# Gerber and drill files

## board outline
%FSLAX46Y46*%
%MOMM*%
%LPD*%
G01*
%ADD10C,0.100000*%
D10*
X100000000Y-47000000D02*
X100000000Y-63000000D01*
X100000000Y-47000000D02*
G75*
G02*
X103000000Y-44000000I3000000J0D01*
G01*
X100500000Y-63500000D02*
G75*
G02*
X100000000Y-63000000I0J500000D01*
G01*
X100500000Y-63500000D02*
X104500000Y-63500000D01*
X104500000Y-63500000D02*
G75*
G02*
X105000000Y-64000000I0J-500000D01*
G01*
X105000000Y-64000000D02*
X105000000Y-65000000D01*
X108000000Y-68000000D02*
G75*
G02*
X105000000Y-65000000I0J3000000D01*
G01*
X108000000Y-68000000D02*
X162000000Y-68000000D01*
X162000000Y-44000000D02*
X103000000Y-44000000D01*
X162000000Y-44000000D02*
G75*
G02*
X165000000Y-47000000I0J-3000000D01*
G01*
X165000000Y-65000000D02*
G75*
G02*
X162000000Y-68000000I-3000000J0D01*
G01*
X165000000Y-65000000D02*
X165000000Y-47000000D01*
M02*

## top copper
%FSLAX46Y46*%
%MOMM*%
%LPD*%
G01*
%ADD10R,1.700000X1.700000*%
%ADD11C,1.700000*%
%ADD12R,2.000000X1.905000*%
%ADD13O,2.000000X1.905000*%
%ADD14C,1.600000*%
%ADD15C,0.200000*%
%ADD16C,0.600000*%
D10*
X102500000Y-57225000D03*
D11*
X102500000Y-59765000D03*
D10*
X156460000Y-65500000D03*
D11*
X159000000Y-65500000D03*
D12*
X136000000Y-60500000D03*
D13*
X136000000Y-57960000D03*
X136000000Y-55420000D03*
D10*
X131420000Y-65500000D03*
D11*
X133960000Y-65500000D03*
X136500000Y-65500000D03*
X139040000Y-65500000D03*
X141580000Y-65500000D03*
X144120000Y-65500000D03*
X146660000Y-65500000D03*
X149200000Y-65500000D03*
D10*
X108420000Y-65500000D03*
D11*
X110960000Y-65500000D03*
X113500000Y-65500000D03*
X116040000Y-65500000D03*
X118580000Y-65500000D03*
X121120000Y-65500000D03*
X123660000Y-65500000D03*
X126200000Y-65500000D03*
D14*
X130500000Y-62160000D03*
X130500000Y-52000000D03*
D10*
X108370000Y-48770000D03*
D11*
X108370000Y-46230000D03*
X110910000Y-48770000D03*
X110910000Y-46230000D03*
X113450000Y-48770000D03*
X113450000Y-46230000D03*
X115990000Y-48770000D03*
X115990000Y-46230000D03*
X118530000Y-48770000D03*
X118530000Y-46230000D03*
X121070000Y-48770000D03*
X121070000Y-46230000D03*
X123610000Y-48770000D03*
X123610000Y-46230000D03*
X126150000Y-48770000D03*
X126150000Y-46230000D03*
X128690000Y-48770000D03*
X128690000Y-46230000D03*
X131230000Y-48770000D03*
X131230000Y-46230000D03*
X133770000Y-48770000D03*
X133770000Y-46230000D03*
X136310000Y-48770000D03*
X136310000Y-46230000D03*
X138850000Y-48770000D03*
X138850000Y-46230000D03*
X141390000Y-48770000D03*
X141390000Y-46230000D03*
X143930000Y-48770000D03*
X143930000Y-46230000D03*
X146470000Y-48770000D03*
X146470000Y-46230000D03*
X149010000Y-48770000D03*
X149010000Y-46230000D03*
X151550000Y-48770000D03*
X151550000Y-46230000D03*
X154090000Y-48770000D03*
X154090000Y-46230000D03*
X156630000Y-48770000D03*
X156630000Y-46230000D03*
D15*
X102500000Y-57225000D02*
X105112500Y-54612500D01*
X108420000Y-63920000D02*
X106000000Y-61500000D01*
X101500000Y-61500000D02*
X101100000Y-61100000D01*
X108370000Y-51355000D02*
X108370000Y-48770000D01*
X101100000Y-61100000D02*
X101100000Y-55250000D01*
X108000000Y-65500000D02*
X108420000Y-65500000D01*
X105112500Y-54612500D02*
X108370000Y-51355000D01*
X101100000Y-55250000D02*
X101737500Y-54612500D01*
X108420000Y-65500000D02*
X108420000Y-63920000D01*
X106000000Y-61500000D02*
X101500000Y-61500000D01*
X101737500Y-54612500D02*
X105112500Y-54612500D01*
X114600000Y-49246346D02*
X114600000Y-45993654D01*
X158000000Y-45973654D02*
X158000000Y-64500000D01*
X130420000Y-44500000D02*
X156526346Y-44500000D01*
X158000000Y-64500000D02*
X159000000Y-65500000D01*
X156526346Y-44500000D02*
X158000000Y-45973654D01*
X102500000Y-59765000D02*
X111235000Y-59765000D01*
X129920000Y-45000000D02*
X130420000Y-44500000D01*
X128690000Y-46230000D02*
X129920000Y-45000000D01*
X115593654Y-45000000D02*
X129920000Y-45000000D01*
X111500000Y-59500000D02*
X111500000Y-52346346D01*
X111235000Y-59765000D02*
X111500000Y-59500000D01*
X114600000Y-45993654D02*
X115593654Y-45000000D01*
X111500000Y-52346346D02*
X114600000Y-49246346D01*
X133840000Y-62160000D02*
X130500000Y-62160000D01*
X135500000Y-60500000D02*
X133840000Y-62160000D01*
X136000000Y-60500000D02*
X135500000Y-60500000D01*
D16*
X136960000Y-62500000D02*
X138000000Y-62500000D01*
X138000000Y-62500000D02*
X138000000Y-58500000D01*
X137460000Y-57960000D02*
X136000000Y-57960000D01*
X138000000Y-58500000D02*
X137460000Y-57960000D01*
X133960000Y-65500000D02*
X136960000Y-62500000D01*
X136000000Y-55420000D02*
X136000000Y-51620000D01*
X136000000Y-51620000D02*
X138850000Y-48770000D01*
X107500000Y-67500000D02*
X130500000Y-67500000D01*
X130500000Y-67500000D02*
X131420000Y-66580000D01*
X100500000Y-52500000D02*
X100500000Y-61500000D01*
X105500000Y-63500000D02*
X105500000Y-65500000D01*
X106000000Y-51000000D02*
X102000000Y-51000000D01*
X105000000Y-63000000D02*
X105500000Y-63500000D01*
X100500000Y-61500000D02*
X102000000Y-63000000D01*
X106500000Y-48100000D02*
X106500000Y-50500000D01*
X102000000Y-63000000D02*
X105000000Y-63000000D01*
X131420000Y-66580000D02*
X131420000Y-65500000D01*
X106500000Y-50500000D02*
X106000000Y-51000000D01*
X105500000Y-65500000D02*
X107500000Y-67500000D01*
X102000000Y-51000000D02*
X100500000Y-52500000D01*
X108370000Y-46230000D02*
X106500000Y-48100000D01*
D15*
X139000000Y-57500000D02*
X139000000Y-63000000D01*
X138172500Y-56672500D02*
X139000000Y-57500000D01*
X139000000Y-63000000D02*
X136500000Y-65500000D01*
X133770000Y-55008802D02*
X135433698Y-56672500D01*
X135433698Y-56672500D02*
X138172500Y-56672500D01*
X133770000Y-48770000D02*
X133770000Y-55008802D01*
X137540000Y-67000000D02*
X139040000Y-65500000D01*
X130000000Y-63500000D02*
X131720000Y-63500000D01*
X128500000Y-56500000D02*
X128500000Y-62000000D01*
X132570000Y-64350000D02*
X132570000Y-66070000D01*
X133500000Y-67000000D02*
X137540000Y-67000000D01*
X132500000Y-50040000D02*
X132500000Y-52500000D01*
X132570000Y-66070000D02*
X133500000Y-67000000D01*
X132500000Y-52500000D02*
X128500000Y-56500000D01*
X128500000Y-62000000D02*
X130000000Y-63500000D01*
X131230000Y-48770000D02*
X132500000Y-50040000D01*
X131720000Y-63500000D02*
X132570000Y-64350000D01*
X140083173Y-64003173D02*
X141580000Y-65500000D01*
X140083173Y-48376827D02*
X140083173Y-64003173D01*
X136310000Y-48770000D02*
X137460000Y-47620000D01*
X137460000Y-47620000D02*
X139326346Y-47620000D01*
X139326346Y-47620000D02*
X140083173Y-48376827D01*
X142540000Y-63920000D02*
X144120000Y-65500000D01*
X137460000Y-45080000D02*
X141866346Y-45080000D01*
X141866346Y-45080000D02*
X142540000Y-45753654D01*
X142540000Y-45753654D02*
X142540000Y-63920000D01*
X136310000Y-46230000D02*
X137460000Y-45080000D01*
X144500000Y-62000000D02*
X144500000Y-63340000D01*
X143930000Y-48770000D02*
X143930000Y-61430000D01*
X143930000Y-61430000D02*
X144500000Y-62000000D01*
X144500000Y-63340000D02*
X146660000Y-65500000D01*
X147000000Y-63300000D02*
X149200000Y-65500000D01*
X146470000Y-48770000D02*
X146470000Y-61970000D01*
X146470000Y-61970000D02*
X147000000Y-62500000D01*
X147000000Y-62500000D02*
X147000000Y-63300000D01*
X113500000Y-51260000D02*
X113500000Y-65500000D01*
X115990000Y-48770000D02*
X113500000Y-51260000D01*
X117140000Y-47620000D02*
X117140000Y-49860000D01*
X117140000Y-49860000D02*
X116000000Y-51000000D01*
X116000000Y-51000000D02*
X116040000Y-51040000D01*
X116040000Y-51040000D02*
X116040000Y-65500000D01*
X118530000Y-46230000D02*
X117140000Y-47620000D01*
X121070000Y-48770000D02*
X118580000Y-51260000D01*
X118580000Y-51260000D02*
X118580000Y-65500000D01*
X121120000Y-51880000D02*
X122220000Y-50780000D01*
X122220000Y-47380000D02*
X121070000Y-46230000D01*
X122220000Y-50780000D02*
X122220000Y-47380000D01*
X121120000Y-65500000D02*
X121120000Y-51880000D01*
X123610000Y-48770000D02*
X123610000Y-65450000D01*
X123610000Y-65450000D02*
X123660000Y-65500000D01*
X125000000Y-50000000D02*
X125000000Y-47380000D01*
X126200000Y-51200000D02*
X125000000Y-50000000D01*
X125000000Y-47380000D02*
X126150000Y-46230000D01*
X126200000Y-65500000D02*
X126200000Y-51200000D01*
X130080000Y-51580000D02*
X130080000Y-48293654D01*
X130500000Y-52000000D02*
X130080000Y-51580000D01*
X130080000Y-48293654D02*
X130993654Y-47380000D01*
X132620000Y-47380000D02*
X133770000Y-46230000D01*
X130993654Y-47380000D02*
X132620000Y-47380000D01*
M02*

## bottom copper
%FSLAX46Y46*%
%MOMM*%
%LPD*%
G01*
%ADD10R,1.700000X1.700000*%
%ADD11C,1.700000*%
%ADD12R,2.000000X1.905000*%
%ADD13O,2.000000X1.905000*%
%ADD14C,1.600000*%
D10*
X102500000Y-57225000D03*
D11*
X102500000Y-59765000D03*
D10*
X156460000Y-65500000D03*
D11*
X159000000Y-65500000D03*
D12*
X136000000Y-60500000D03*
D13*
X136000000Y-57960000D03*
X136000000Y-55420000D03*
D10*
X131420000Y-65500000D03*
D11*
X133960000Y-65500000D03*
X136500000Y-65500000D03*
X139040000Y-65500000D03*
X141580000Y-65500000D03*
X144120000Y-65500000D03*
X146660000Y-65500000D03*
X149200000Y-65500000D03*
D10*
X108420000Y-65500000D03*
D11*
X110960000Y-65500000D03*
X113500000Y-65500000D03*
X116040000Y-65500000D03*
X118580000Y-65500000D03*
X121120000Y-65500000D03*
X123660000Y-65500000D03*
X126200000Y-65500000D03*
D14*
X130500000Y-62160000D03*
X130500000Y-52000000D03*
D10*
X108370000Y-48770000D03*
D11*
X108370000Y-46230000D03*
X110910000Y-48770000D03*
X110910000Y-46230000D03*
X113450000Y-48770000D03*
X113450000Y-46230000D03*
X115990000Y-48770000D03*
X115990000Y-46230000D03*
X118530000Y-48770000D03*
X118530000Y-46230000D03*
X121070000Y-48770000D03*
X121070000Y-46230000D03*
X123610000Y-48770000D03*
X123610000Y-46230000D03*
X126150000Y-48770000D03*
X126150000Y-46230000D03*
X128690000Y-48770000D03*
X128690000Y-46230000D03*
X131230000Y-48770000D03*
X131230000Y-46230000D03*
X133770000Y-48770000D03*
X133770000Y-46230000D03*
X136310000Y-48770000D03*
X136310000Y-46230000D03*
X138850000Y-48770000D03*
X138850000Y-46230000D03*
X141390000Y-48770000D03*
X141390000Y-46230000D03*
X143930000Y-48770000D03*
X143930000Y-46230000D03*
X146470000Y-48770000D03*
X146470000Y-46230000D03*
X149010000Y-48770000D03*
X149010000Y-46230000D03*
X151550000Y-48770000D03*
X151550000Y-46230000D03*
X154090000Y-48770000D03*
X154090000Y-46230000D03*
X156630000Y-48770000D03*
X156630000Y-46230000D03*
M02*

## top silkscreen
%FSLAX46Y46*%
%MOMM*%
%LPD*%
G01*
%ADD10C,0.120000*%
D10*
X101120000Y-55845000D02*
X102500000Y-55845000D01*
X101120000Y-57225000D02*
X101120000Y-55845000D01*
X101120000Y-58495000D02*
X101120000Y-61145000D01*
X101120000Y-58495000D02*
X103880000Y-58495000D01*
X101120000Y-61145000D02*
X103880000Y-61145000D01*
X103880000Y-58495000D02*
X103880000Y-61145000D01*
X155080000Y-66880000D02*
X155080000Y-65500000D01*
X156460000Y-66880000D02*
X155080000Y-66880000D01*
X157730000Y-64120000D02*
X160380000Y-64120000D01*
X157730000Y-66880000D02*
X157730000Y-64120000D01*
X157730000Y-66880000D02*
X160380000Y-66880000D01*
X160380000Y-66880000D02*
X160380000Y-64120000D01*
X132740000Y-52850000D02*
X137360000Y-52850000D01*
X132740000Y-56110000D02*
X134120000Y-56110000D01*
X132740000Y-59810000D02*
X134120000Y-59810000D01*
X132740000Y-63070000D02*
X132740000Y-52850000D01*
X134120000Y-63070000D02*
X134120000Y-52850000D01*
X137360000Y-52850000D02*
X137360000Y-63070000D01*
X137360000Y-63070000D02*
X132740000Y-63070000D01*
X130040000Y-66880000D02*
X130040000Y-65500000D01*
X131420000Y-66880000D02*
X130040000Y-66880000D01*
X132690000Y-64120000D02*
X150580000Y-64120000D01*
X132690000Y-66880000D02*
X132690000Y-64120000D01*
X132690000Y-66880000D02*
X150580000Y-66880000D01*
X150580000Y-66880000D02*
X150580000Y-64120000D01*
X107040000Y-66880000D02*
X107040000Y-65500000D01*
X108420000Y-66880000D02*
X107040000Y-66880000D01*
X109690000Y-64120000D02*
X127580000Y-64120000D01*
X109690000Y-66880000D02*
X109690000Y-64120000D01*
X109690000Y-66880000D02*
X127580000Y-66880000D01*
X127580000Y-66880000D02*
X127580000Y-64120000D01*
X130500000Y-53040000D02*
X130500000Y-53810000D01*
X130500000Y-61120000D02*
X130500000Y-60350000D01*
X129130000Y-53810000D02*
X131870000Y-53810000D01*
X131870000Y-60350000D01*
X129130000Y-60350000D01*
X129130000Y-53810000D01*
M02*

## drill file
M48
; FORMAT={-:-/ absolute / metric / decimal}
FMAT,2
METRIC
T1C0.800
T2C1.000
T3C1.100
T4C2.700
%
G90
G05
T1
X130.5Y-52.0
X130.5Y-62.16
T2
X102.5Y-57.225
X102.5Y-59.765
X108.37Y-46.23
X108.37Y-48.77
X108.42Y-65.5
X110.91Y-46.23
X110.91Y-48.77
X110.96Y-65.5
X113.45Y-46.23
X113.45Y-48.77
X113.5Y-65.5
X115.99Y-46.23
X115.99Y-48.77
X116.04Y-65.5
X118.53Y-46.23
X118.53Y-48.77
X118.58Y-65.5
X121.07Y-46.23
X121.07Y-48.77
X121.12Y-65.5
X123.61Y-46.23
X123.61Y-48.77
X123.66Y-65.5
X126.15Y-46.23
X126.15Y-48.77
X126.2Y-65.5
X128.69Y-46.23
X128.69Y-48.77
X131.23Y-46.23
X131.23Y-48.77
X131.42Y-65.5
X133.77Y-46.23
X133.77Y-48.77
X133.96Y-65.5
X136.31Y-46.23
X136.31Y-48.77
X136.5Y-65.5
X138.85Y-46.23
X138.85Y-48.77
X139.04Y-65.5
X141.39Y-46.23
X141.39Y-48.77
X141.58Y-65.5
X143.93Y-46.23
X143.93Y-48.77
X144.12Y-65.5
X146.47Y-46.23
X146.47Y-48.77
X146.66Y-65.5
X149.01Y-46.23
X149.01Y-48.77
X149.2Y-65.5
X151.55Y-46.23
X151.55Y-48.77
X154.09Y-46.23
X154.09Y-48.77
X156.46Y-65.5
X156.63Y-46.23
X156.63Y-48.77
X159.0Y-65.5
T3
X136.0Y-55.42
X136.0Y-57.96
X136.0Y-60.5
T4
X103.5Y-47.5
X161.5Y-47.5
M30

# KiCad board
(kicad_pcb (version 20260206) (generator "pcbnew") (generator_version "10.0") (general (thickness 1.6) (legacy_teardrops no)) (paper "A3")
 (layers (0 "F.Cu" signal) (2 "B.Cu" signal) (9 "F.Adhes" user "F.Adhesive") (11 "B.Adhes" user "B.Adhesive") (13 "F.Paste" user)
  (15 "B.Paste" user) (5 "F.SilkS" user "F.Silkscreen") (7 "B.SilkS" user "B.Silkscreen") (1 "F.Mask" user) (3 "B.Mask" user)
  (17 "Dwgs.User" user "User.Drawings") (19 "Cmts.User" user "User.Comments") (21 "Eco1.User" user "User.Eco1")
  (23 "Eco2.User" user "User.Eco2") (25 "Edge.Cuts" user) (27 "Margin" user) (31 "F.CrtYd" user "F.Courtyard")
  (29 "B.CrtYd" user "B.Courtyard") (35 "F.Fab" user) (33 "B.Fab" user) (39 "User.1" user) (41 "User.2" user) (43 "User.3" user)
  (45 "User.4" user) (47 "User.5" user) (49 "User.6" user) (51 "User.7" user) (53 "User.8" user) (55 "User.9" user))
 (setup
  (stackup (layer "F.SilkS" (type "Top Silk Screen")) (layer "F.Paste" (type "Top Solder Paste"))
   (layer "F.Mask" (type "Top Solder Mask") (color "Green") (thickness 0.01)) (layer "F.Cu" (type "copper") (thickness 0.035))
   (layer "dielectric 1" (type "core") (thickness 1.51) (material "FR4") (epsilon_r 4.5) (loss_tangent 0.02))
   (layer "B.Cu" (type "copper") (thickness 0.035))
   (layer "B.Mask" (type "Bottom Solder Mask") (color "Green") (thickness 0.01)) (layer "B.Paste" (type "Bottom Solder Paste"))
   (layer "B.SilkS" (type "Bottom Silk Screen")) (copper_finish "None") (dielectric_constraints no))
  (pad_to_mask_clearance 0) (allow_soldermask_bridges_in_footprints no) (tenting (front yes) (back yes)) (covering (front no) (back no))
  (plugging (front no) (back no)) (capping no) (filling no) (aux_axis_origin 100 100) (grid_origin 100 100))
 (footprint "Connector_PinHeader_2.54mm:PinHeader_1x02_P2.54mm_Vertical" (layer "F.Cu") (at 102.5 57.225)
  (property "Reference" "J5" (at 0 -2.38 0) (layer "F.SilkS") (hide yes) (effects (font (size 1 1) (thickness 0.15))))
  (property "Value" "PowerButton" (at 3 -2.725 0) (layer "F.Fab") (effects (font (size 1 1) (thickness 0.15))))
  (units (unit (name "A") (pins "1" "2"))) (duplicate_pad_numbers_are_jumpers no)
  (fp_line (start -1.38 -1.38) (end 0 -1.38) (stroke (width 0.12) (type solid)) (layer "F.SilkS"))
  (fp_line (start -1.38 0) (end -1.38 -1.38) (stroke (width 0.12) (type solid)) (layer "F.SilkS"))
  (fp_line (start -1.38 1.27) (end -1.38 3.92) (stroke (width 0.12) (type solid)) (layer "F.SilkS"))
  (fp_line (start -1.38 1.27) (end 1.38 1.27) (stroke (width 0.12) (type solid)) (layer "F.SilkS"))
  (fp_line (start -1.38 3.92) (end 1.38 3.92) (stroke (width 0.12) (type solid)) (layer "F.SilkS"))
  (fp_line (start 1.38 1.27) (end 1.38 3.92) (stroke (width 0.12) (type solid)) (layer "F.SilkS"))
  (pad "1" thru_hole rect (at 0 0) (size 1.7 1.7) (drill 1) (layers "*.Cu" "*.Mask") (remove_unused_layers no) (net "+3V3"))
  (pad "2" thru_hole circle (at 0 2.54) (size 1.7 1.7) (drill 1) (layers "*.Cu" "*.Mask") (remove_unused_layers no) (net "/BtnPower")))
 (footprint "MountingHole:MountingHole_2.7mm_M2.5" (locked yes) (layer "F.Cu") (at 161.5 47.5)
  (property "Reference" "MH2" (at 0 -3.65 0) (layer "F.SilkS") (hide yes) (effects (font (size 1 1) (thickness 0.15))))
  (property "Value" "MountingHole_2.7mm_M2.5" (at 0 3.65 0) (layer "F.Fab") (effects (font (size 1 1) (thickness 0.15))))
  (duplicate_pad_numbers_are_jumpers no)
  (pad "" np_thru_hole circle (at 0 0) (size 2.7 2.7) (drill 2.7) (layers "*.Cu" "*.Mask")))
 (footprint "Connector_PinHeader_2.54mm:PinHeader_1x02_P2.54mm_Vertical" (layer "F.Cu") (at 156.46 65.5 90)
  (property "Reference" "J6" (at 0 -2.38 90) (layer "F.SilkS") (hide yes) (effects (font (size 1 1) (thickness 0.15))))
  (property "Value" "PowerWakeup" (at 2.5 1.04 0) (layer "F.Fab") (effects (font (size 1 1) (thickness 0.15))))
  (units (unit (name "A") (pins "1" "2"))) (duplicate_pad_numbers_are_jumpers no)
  (fp_line (start -1.38 -1.38) (end 0 -1.38) (stroke (width 0.12) (type solid)) (layer "F.SilkS"))
  (fp_line (start -1.38 0) (end -1.38 -1.38) (stroke (width 0.12) (type solid)) (layer "F.SilkS"))
  (fp_line (start 1.38 1.27) (end 1.38 3.92) (stroke (width 0.12) (type solid)) (layer "F.SilkS"))
  (fp_line (start -1.38 1.27) (end 1.38 1.27) (stroke (width 0.12) (type solid)) (layer "F.SilkS"))
  (fp_line (start -1.38 1.27) (end -1.38 3.92) (stroke (width 0.12) (type solid)) (layer "F.SilkS"))
  (fp_line (start -1.38 3.92) (end 1.38 3.92) (stroke (width 0.12) (type solid)) (layer "F.SilkS"))
  (pad "1" thru_hole rect (at 0 0 90) (size 1.7 1.7) (drill 1) (layers "*.Cu" "*.Mask") (remove_unused_layers no)
   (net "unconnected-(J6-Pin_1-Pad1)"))
  (pad "2" thru_hole circle (at 0 2.54 90) (size 1.7 1.7) (drill 1) (layers "*.Cu" "*.Mask") (remove_unused_layers no) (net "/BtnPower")))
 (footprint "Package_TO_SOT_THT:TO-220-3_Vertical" (layer "F.Cu") (at 136 60.5 90)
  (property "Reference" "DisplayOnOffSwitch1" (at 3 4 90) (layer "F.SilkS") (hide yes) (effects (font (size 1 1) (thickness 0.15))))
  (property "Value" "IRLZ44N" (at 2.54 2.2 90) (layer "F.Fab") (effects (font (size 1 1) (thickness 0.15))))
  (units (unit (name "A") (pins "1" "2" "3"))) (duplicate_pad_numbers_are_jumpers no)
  (fp_line (start 7.65 -3.26) (end 7.65 1.36) (stroke (width 0.12) (type solid)) (layer "F.SilkS"))
  (fp_line (start 4.39 -3.26) (end 4.39 -1.88) (stroke (width 0.12) (type solid)) (layer "F.SilkS"))
  (fp_line (start 0.69 -3.26) (end 0.69 -1.88) (stroke (width 0.12) (type solid)) (layer "F.SilkS"))
  (fp_line (start -2.57 -3.26) (end 7.65 -3.26) (stroke (width 0.12) (type solid)) (layer "F.SilkS"))
  (fp_line (start -2.57 -1.88) (end 7.65 -1.88) (stroke (width 0.12) (type solid)) (layer "F.SilkS"))
  (fp_line (start 7.65 1.36) (end -2.57 1.36) (stroke (width 0.12) (type solid)) (layer "F.SilkS"))
  (fp_line (start -2.57 1.36) (end -2.57 -3.26) (stroke (width 0.12) (type solid)) (layer "F.SilkS"))
  (pad "1" thru_hole rect (at 0 0 90) (size 1.905 2) (drill 1.1) (layers "*.Cu" "*.Mask") (remove_unused_layers no)
   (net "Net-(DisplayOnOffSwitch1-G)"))
  (pad "2" thru_hole oval (at 2.54 0 90) (size 1.905 2) (drill 1.1) (layers "*.Cu" "*.Mask") (remove_unused_layers no) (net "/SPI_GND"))
  (pad "3" thru_hole oval (at 5.08 0 90) (size 1.905 2) (drill 1.1) (layers "*.Cu" "*.Mask") (remove_unused_layers no) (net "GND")))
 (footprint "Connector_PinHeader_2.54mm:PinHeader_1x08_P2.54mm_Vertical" (layer "F.Cu") (at 131.42 65.5 90)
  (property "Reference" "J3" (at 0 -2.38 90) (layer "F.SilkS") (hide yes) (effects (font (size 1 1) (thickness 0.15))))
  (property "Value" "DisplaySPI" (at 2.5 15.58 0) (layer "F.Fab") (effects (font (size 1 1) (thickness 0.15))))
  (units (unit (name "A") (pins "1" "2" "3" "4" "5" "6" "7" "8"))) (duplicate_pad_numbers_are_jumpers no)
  (fp_line (start -1.38 -1.38) (end 0 -1.38) (stroke (width 0.12) (type solid)) (layer "F.SilkS"))
  (fp_line (start -1.38 0) (end -1.38 -1.38) (stroke (width 0.12) (type solid)) (layer "F.SilkS"))
  (fp_line (start 1.38 1.27) (end 1.38 19.16) (stroke (width 0.12) (type solid)) (layer "F.SilkS"))
  (fp_line (start -1.38 1.27) (end 1.38 1.27) (stroke (width 0.12) (type solid)) (layer "F.SilkS"))
  (fp_line (start -1.38 1.27) (end -1.38 19.16) (stroke (width 0.12) (type solid)) (layer "F.SilkS"))
  (fp_line (start -1.38 19.16) (end 1.38 19.16) (stroke (width 0.12) (type solid)) (layer "F.SilkS"))
  (pad "1" thru_hole rect (at 0 0 90) (size 1.7 1.7) (drill 1) (layers "*.Cu" "*.Mask") (remove_unused_layers no) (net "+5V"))
  (pad "2" thru_hole circle (at 0 2.54 90) (size 1.7 1.7) (drill 1) (layers "*.Cu" "*.Mask") (remove_unused_layers no) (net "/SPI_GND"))
  (pad "3" thru_hole circle (at 0 5.08 90) (size 1.7 1.7) (drill 1) (layers "*.Cu" "*.Mask") (remove_unused_layers no)
   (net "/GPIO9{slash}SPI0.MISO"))
  (pad "4" thru_hole circle (at 0 7.62 90) (size 1.7 1.7) (drill 1) (layers "*.Cu" "*.Mask") (remove_unused_layers no)
   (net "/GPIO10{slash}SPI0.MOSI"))
  (pad "5" thru_hole circle (at 0 10.16 90) (size 1.7 1.7) (drill 1) (layers "*.Cu" "*.Mask") (remove_unused_layers no)
   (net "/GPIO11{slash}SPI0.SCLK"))
  (pad "6" thru_hole circle (at 0 12.7 90) (size 1.7 1.7) (drill 1) (layers "*.Cu" "*.Mask") (remove_unused_layers no)
   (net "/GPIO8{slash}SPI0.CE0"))
  (pad "7" thru_hole circle (at 0 15.24 90) (size 1.7 1.7) (drill 1) (layers "*.Cu" "*.Mask") (remove_unused_layers no) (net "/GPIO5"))
  (pad "8" thru_hole circle (at 0 17.78 90) (size 1.7 1.7) (drill 1) (layers "*.Cu" "*.Mask") (remove_unused_layers no) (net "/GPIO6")))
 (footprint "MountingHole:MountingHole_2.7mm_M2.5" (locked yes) (layer "F.Cu") (at 103.5 47.5)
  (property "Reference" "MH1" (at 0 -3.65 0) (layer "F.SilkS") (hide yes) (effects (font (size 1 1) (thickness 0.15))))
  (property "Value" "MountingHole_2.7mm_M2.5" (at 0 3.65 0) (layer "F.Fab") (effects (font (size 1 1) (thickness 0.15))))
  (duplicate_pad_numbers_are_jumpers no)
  (pad "" np_thru_hole circle (at 0 0) (size 2.7 2.7) (drill 2.7) (layers "*.Cu" "*.Mask")))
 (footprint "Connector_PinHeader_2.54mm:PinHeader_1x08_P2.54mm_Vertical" (layer "F.Cu") (at 108.42 65.5 90)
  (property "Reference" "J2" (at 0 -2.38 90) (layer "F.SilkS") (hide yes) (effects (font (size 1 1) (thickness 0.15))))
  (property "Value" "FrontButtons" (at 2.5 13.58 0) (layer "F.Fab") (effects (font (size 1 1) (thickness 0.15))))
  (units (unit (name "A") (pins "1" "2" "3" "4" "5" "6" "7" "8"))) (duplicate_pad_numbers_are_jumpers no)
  (fp_line (start -1.38 -1.38) (end 0 -1.38) (stroke (width 0.12) (type solid)) (layer "F.SilkS"))
  (fp_line (start -1.38 0) (end -1.38 -1.38) (stroke (width 0.12) (type solid)) (layer "F.SilkS"))
  (fp_line (start 1.38 1.27) (end 1.38 19.16) (stroke (width 0.12) (type solid)) (layer "F.SilkS"))
  (fp_line (start -1.38 1.27) (end 1.38 1.27) (stroke (width 0.12) (type solid)) (layer "F.SilkS"))
  (fp_line (start -1.38 1.27) (end -1.38 19.16) (stroke (width 0.12) (type solid)) (layer "F.SilkS"))
  (fp_line (start -1.38 19.16) (end 1.38 19.16) (stroke (width 0.12) (type solid)) (layer "F.SilkS"))
  (pad "1" thru_hole rect (at 0 0 90) (size 1.7 1.7) (drill 1) (layers "*.Cu" "*.Mask") (remove_unused_layers no) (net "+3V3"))
  (pad "2" thru_hole circle (at 0 2.54 90) (size 1.7 1.7) (drill 1) (layers "*.Cu" "*.Mask") (remove_unused_layers no)
   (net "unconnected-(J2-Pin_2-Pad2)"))
  (pad "3" thru_hole circle (at 0 5.08 90) (size 1.7 1.7) (drill 1) (layers "*.Cu" "*.Mask") (remove_unused_layers no) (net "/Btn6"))
  (pad "4" thru_hole circle (at 0 7.62 90) (size 1.7 1.7) (drill 1) (layers "*.Cu" "*.Mask") (remove_unused_layers no) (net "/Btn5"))
  (pad "5" thru_hole circle (at 0 10.16 90) (size 1.7 1.7) (drill 1) (layers "*.Cu" "*.Mask") (remove_unused_layers no) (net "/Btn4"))
  (pad "6" thru_hole circle (at 0 12.7 90) (size 1.7 1.7) (drill 1) (layers "*.Cu" "*.Mask") (remove_unused_layers no) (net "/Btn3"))
  (pad "7" thru_hole circle (at 0 15.24 90) (size 1.7 1.7) (drill 1) (layers "*.Cu" "*.Mask") (remove_unused_layers no) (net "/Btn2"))
  (pad "8" thru_hole circle (at 0 17.78 90) (size 1.7 1.7) (drill 1) (layers "*.Cu" "*.Mask") (remove_unused_layers no) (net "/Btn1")))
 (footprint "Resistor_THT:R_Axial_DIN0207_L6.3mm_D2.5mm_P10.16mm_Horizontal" (layer "F.Cu") (at 130.5 62.16 90)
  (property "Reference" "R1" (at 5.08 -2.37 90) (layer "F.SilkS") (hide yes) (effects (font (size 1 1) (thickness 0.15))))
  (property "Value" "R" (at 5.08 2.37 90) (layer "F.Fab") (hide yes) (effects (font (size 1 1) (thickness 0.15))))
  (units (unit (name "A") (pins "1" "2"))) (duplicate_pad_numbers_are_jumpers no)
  (fp_line (start 9.12 0) (end 8.35 0) (stroke (width 0.12) (type solid)) (layer "F.SilkS"))
  (fp_line (start 1.04 0) (end 1.81 0) (stroke (width 0.12) (type solid)) (layer "F.SilkS"))
  (fp_rect (start 1.81 -1.37) (end 8.35 1.37) (stroke (width 0.12) (type solid)) (fill no) (layer "F.SilkS"))
  (pad "1" thru_hole circle (at 0 0 90) (size 1.6 1.6) (drill 0.8) (layers "*.Cu" "*.Mask") (remove_unused_layers no)
   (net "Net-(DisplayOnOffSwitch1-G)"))
  (pad "2" thru_hole circle (at 10.16 0 90) (size 1.6 1.6) (drill 0.8) (layers "*.Cu" "*.Mask") (remove_unused_layers no)
   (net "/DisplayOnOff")))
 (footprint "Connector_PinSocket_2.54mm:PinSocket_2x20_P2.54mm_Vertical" (layer "B.Cu") (at 108.37 48.77 -90)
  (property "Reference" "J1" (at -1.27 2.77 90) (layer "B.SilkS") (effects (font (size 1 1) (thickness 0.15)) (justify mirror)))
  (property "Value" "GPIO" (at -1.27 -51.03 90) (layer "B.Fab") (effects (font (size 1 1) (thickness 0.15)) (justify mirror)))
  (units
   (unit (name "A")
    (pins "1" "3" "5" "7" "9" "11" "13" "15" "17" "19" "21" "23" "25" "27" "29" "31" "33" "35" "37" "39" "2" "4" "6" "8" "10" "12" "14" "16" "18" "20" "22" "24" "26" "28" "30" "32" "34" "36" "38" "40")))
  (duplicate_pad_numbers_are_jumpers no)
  (pad "1" thru_hole rect (at 0 0 270) (size 1.7 1.7) (drill 1) (layers "*.Cu" "*.Mask") (remove_unused_layers no) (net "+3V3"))
  (pad "2" thru_hole circle (at -2.54 0 270) (size 1.7 1.7) (drill 1) (layers "*.Cu" "*.Mask") (remove_unused_layers no) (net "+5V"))
  (pad "3" thru_hole circle (at 0 -2.54 270) (size 1.7 1.7) (drill 1) (layers "*.Cu" "*.Mask") (remove_unused_layers no)
   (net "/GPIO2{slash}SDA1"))
  (pad "4" thru_hole circle (at -2.54 -2.54 270) (size 1.7 1.7) (drill 1) (layers "*.Cu" "*.Mask") (remove_unused_layers no) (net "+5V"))
  (pad "5" thru_hole circle (at 0 -5.08 270) (size 1.7 1.7) (drill 1) (layers "*.Cu" "*.Mask") (remove_unused_layers no)
   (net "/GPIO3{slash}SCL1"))
  (pad "6" thru_hole circle (at -2.54 -5.08 270) (size 1.7 1.7) (drill 1) (layers "*.Cu" "*.Mask") (remove_unused_layers no) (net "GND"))
  (pad "7" thru_hole circle (at 0 -7.62 270) (size 1.7 1.7) (drill 1) (layers "*.Cu" "*.Mask") (remove_unused_layers no) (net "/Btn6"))
  (pad "8" thru_hole circle (at -2.54 -7.62 270) (size 1.7 1.7) (drill 1) (layers "*.Cu" "*.Mask") (remove_unused_layers no)
   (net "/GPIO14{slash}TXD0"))
  (pad "9" thru_hole circle (at 0 -10.16 270) (size 1.7 1.7) (drill 1) (layers "*.Cu" "*.Mask") (remove_unused_layers no) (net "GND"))
  (pad "10" thru_hole circle (at -2.54 -10.16 270) (size 1.7 1.7) (drill 1) (layers "*.Cu" "*.Mask") (remove_unused_layers no) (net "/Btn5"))
  (pad "11" thru_hole circle (at 0 -12.7 270) (size 1.7 1.7) (drill 1) (layers "*.Cu" "*.Mask") (remove_unused_layers no) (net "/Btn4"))
  (pad "12" thru_hole circle (at -2.54 -12.7 270) (size 1.7 1.7) (drill 1) (layers "*.Cu" "*.Mask") (remove_unused_layers no) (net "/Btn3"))
  (pad "13" thru_hole circle (at 0 -15.24 270) (size 1.7 1.7) (drill 1) (layers "*.Cu" "*.Mask") (remove_unused_layers no) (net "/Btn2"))
  (pad "14" thru_hole circle (at -2.54 -15.24 270) (size 1.7 1.7) (drill 1) (layers "*.Cu" "*.Mask") (remove_unused_layers no) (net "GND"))
  (pad "15" thru_hole circle (at 0 -17.78 270) (size 1.7 1.7) (drill 1) (layers "*.Cu" "*.Mask") (remove_unused_layers no) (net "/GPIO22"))
  (pad "16" thru_hole circle (at -2.54 -17.78 270) (size 1.7 1.7) (drill 1) (layers "*.Cu" "*.Mask") (remove_unused_layers no) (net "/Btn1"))
  (pad "17" thru_hole circle (at 0 -20.32 270) (size 1.7 1.7) (drill 1) (layers "*.Cu" "*.Mask") (remove_unused_layers no) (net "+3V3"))
  (pad "18" thru_hole circle (at -2.54 -20.32 270) (size 1.7 1.7) (drill 1) (layers "*.Cu" "*.Mask") (remove_unused_layers no)
   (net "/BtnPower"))
  (pad "19" thru_hole circle (at 0 -22.86 270) (size 1.7 1.7) (drill 1) (layers "*.Cu" "*.Mask") (remove_unused_layers no)
   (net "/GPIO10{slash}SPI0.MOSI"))
  (pad "20" thru_hole circle (at -2.54 -22.86 270) (size 1.7 1.7) (drill 1) (layers "*.Cu" "*.Mask") (remove_unused_layers no) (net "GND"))
  (pad "21" thru_hole circle (at 0 -25.4 270) (size 1.7 1.7) (drill 1) (layers "*.Cu" "*.Mask") (remove_unused_layers no)
   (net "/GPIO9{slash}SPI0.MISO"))
  (pad "22" thru_hole circle (at -2.54 -25.4 270) (size 1.7 1.7) (drill 1) (layers "*.Cu" "*.Mask") (remove_unused_layers no)
   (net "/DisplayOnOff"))
  (pad "23" thru_hole circle (at 0 -27.94 270) (size 1.7 1.7) (drill 1) (layers "*.Cu" "*.Mask") (remove_unused_layers no)
   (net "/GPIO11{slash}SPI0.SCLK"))
  (pad "24" thru_hole circle (at -2.54 -27.94 270) (size 1.7 1.7) (drill 1) (layers "*.Cu" "*.Mask") (remove_unused_layers no)
   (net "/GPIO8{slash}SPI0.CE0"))
  (pad "25" thru_hole circle (at 0 -30.48 270) (size 1.7 1.7) (drill 1) (layers "*.Cu" "*.Mask") (remove_unused_layers no) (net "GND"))
  (pad "26" thru_hole circle (at -2.54 -30.48 270) (size 1.7 1.7) (drill 1) (layers "*.Cu" "*.Mask") (remove_unused_layers no)
   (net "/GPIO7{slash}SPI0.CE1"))
  (pad "27" thru_hole circle (at 0 -33.02 270) (size 1.7 1.7) (drill 1) (layers "*.Cu" "*.Mask") (remove_unused_layers no) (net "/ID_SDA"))
  (pad "28" thru_hole circle (at -2.54 -33.02 270) (size 1.7 1.7) (drill 1) (layers "*.Cu" "*.Mask") (remove_unused_layers no)
   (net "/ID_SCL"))
  (pad "29" thru_hole circle (at 0 -35.56 270) (size 1.7 1.7) (drill 1) (layers "*.Cu" "*.Mask") (remove_unused_layers no) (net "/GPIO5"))
  (pad "30" thru_hole circle (at -2.54 -35.56 270) (size 1.7 1.7) (drill 1) (layers "*.Cu" "*.Mask") (remove_unused_layers no) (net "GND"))
  (pad "31" thru_hole circle (at 0 -38.1 270) (size 1.7 1.7) (drill 1) (layers "*.Cu" "*.Mask") (remove_unused_layers no) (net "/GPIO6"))
  (pad "32" thru_hole circle (at -2.54 -38.1 270) (size 1.7 1.7) (drill 1) (layers "*.Cu" "*.Mask") (remove_unused_layers no)
   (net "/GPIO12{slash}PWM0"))
  (pad "33" thru_hole circle (at 0 -40.64 270) (size 1.7 1.7) (drill 1) (layers "*.Cu" "*.Mask") (remove_unused_layers no)
   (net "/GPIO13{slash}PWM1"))
  (pad "34" thru_hole circle (at -2.54 -40.64 270) (size 1.7 1.7) (drill 1) (layers "*.Cu" "*.Mask") (remove_unused_layers no) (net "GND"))
  (pad "35" thru_hole circle (at 0 -43.18 270) (size 1.7 1.7) (drill 1) (layers "*.Cu" "*.Mask") (remove_unused_layers no)
   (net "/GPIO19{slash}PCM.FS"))
  (pad "36" thru_hole circle (at -2.54 -43.18 270) (size 1.7 1.7) (drill 1) (layers "*.Cu" "*.Mask") (remove_unused_layers no)
   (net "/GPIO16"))
  (pad "37" thru_hole circle (at 0 -45.72 270) (size 1.7 1.7) (drill 1) (layers "*.Cu" "*.Mask") (remove_unused_layers no) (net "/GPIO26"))
  (pad "38" thru_hole circle (at -2.54 -45.72 270) (size 1.7 1.7) (drill 1) (layers "*.Cu" "*.Mask") (remove_unused_layers no)
   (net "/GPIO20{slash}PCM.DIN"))
  (pad "39" thru_hole circle (at 0 -48.26 270) (size 1.7 1.7) (drill 1) (layers "*.Cu" "*.Mask") (remove_unused_layers no) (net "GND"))
  (pad "40" thru_hole circle (at -2.54 -48.26 270) (size 1.7 1.7) (drill 1) (layers "*.Cu" "*.Mask") (remove_unused_layers no)
   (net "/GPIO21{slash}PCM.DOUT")))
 (gr_line (start 100 47) (end 100 63) (stroke (width 0.1) (type solid)) (layer "Edge.Cuts"))
 (gr_arc (start 100 47) (mid 100.87868 44.87868) (end 103 44) (stroke (width 0.1) (type solid)) (layer "Edge.Cuts"))
 (gr_arc (start 100.5 63.5) (mid 100.146447 63.353553) (end 100 63) (stroke (width 0.1) (type solid)) (layer "Edge.Cuts"))
 (gr_line (start 100.5 63.5) (end 104.5 63.5) (stroke (width 0.1) (type solid)) (layer "Edge.Cuts"))
 (gr_arc (start 104.5 63.5) (mid 104.853553 63.646447) (end 105 64) (stroke (width 0.1) (type solid)) (layer "Edge.Cuts"))
 (gr_line (start 105 64) (end 105 65) (stroke (width 0.1) (type solid)) (layer "Edge.Cuts"))
 (gr_arc (start 108 68) (mid 105.87868 67.12132) (end 105 65) (stroke (width 0.1) (type solid)) (layer "Edge.Cuts"))
 (gr_line (start 108 68) (end 162 68) (stroke (width 0.1) (type solid)) (layer "Edge.Cuts"))
 (gr_line (start 162 44) (end 103 44) (stroke (width 0.1) (type solid)) (layer "Edge.Cuts"))
 (gr_arc (start 162 44) (mid 164.12132 44.87868) (end 165 47) (stroke (width 0.1) (type solid)) (layer "Edge.Cuts"))
 (gr_arc (start 165 65) (mid 164.12132 67.12132) (end 162 68) (stroke (width 0.1) (type solid)) (layer "Edge.Cuts"))
 (gr_line (start 165 65) (end 165 47) (stroke (width 0.1) (type solid)) (layer "Edge.Cuts"))
 (segment (start 102.5 57.225) (end 105.1125 54.6125) (width 0.2) (layer "F.Cu") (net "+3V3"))
 (segment (start 108.42 63.92) (end 106 61.5) (width 0.2) (layer "F.Cu") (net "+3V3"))
 (segment (start 101.5 61.5) (end 101.1 61.1) (width 0.2) (layer "F.Cu") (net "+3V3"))
 (segment (start 108.37 51.355) (end 108.37 48.77) (width 0.2) (layer "F.Cu") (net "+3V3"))
 (segment (start 101.1 61.1) (end 101.1 55.25) (width 0.2) (layer "F.Cu") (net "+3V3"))
 (segment (start 108 65.5) (end 108.42 65.5) (width 0.2) (layer "F.Cu") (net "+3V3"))
 (segment (start 105.1125 54.6125) (end 108.37 51.355) (width 0.2) (layer "F.Cu") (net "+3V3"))
 (segment (start 101.1 55.25) (end 101.7375 54.6125) (width 0.2) (layer "F.Cu") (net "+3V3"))
 (segment (start 108.42 65.5) (end 108.42 63.92) (width 0.2) (layer "F.Cu") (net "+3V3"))
 (segment (start 106 61.5) (end 101.5 61.5) (width 0.2) (layer "F.Cu") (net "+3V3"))
 (segment (start 101.7375 54.6125) (end 105.1125 54.6125) (width 0.2) (layer "F.Cu") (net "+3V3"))
 (segment (start 114.6 49.246346) (end 114.6 45.993654) (width 0.2) (layer "F.Cu") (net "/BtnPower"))
 (segment (start 158 45.973654) (end 158 64.5) (width 0.2) (layer "F.Cu") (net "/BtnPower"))
 (segment (start 130.42 44.5) (end 156.526346 44.5) (width 0.2) (layer "F.Cu") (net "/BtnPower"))
 (segment (start 158 64.5) (end 159 65.5) (width 0.2) (layer "F.Cu") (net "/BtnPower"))
 (segment (start 156.526346 44.5) (end 158 45.973654) (width 0.2) (layer "F.Cu") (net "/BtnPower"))
 (segment (start 102.5 59.765) (end 111.235 59.765) (width 0.2) (layer "F.Cu") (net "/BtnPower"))
 (segment (start 129.92 45) (end 130.42 44.5) (width 0.2) (layer "F.Cu") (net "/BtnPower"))
 (segment (start 128.69 46.23) (end 129.92 45) (width 0.2) (layer "F.Cu") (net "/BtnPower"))
 (segment (start 115.593654 45) (end 129.92 45) (width 0.2) (layer "F.Cu") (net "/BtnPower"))
 (segment (start 111.5 59.5) (end 111.5 52.346346) (width 0.2) (layer "F.Cu") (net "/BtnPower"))
 (segment (start 111.235 59.765) (end 111.5 59.5) (width 0.2) (layer "F.Cu") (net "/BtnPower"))
 (segment (start 114.6 45.993654) (end 115.593654 45) (width 0.2) (layer "F.Cu") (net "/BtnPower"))
 (segment (start 111.5 52.346346) (end 114.6 49.246346) (width 0.2) (layer "F.Cu") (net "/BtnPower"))
 (segment (start 133.84 62.16) (end 130.5 62.16) (width 0.2) (layer "F.Cu") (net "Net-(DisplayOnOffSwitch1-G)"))
 (segment (start 135.5 60.5) (end 133.84 62.16) (width 0.2) (layer "F.Cu") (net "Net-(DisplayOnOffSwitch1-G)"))
 (segment (start 136 60.5) (end 135.5 60.5) (width 0.2) (layer "F.Cu") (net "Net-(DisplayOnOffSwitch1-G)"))
 (segment (start 136.96 62.5) (end 138 62.5) (width 0.6) (layer "F.Cu") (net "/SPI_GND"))
 (segment (start 138 62.5) (end 138 58.5) (width 0.6) (layer "F.Cu") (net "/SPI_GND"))
 (segment (start 137.46 57.96) (end 136 57.96) (width 0.6) (layer "F.Cu") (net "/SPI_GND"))
 (segment (start 138 58.5) (end 137.46 57.96) (width 0.6) (layer "F.Cu") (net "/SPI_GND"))
 (segment (start 133.96 65.5) (end 136.96 62.5) (width 0.6) (layer "F.Cu") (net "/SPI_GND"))
 (segment (start 136 55.42) (end 136 51.62) (width 0.6) (layer "F.Cu") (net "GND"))
 (segment (start 136 51.62) (end 138.85 48.77) (width 0.6) (layer "F.Cu") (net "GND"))
 (segment (start 107.5 67.5) (end 130.5 67.5) (width 0.6) (layer "F.Cu") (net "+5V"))
 (segment (start 130.5 67.5) (end 131.42 66.58) (width 0.6) (layer "F.Cu") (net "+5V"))
 (segment (start 100.5 52.5) (end 100.5 61.5) (width 0.6) (layer "F.Cu") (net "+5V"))
 (segment (start 105.5 63.5) (end 105.5 65.5) (width 0.6) (layer "F.Cu") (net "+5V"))
 (segment (start 106 51) (end 102 51) (width 0.6) (layer "F.Cu") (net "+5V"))
 (segment (start 105 63) (end 105.5 63.5) (width 0.6) (layer "F.Cu") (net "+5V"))
 (segment (start 100.5 61.5) (end 102 63) (width 0.6) (layer "F.Cu") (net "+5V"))
 (segment (start 106.5 48.1) (end 106.5 50.5) (width 0.6) (layer "F.Cu") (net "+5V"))
 (segment (start 102 63) (end 105 63) (width 0.6) (layer "F.Cu") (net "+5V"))
 (segment (start 131.42 66.58) (end 131.42 65.5) (width 0.6) (layer "F.Cu") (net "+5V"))
 (segment (start 106.5 50.5) (end 106 51) (width 0.6) (layer "F.Cu") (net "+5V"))
 (segment (start 105.5 65.5) (end 107.5 67.5) (width 0.6) (layer "F.Cu") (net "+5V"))
 (segment (start 102 51) (end 100.5 52.5) (width 0.6) (layer "F.Cu") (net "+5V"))
 (segment (start 108.37 46.23) (end 106.5 48.1) (width 0.6) (layer "F.Cu") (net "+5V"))
 (segment (start 139 57.5) (end 139 63) (width 0.2) (layer "F.Cu") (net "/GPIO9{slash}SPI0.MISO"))
 (segment (start 138.1725 56.6725) (end 139 57.5) (width 0.2) (layer "F.Cu") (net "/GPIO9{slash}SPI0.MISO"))
 (segment (start 139 63) (end 136.5 65.5) (width 0.2) (layer "F.Cu") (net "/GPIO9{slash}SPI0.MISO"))
 (segment (start 133.77 55.008802) (end 135.433698 56.6725) (width 0.2) (layer "F.Cu") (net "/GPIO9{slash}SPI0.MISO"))
 (segment (start 135.433698 56.6725) (end 138.1725 56.6725) (width 0.2) (layer "F.Cu") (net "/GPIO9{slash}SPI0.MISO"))
 (segment (start 133.77 48.77) (end 133.77 55.008802) (width 0.2) (layer "F.Cu") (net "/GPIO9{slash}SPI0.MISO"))
 (segment (start 137.54 67) (end 139.04 65.5) (width 0.2) (layer "F.Cu") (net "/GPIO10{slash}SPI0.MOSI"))
 (segment (start 130 63.5) (end 131.72 63.5) (width 0.2) (layer "F.Cu") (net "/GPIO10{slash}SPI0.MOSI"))
 (segment (start 128.5 56.5) (end 128.5 62) (width 0.2) (layer "F.Cu") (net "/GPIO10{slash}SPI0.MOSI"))
 (segment (start 132.57 64.35) (end 132.57 66.07) (width 0.2) (layer "F.Cu") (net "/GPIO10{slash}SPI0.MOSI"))
 (segment (start 133.5 67) (end 137.54 67) (width 0.2) (layer "F.Cu") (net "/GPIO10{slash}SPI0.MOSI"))
 (segment (start 132.5 50.04) (end 132.5 52.5) (width 0.2) (layer "F.Cu") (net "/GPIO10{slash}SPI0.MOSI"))
 (segment (start 132.57 66.07) (end 133.5 67) (width 0.2) (layer "F.Cu") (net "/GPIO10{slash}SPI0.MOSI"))
 (segment (start 132.5 52.5) (end 128.5 56.5) (width 0.2) (layer "F.Cu") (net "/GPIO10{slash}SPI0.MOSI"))
 (segment (start 128.5 62) (end 130 63.5) (width 0.2) (layer "F.Cu") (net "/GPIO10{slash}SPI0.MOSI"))
 (segment (start 131.23 48.77) (end 132.5 50.04) (width 0.2) (layer "F.Cu") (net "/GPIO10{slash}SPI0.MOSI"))
 (segment (start 131.72 63.5) (end 132.57 64.35) (width 0.2) (layer "F.Cu") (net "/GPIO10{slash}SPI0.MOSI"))
 (segment (start 140.083173 64.003173) (end 141.58 65.5) (width 0.2) (layer "F.Cu") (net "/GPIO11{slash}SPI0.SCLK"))
 (segment (start 140.083173 48.376827) (end 140.083173 64.003173) (width 0.2) (layer "F.Cu") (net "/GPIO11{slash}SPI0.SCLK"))
 (segment (start 136.31 48.77) (end 137.46 47.62) (width 0.2) (layer "F.Cu") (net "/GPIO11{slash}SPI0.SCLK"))
 (segment (start 137.46 47.62) (end 139.326346 47.62) (width 0.2) (layer "F.Cu") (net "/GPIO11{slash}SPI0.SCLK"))
 (segment (start 139.326346 47.62) (end 140.083173 48.376827) (width 0.2) (layer "F.Cu") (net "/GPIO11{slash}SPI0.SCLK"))
 (segment (start 142.54 63.92) (end 144.12 65.5) (width 0.2) (layer "F.Cu") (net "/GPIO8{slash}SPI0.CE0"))
 (segment (start 137.46 45.08) (end 141.866346 45.08) (width 0.2) (layer "F.Cu") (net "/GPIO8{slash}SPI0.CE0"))
 (segment (start 141.866346 45.08) (end 142.54 45.753654) (width 0.2) (layer "F.Cu") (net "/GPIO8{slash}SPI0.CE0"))
 (segment (start 142.54 45.753654) (end 142.54 63.92) (width 0.2) (layer "F.Cu") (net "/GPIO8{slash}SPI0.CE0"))
 (segment (start 136.31 46.23) (end 137.46 45.08) (width 0.2) (layer "F.Cu") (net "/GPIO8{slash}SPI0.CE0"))
 (segment (start 144.5 62) (end 144.5 63.34) (width 0.2) (layer "F.Cu") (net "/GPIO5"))
 (segment (start 143.93 48.77) (end 143.93 61.43) (width 0.2) (layer "F.Cu") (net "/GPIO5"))
 (segment (start 143.93 61.43) (end 144.5 62) (width 0.2) (layer "F.Cu") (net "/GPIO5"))
 (segment (start 144.5 63.34) (end 146.66 65.5) (width 0.2) (layer "F.Cu") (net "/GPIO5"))
 (segment (start 147 63.3) (end 149.2 65.5) (width 0.2) (layer "F.Cu") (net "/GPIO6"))
 (segment (start 146.47 48.77) (end 146.47 61.97) (width 0.2) (layer "F.Cu") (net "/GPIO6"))
 (segment (start 146.47 61.97) (end 147 62.5) (width 0.2) (layer "F.Cu") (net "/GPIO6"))
 (segment (start 147 62.5) (end 147 63.3) (width 0.2) (layer "F.Cu") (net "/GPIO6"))
 (segment (start 113.5 51.26) (end 113.5 65.5) (width 0.2) (layer "F.Cu") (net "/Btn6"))
 (segment (start 115.99 48.77) (end 113.5 51.26) (width 0.2) (layer "F.Cu") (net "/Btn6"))
 (segment (start 117.14 47.62) (end 117.14 49.86) (width 0.2) (layer "F.Cu") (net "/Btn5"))
 (segment (start 117.14 49.86) (end 116 51) (width 0.2) (layer "F.Cu") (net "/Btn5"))
 (segment (start 116 51) (end 116.04 51.04) (width 0.2) (layer "F.Cu") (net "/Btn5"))
 (segment (start 116.04 51.04) (end 116.04 65.5) (width 0.2) (layer "F.Cu") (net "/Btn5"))
 (segment (start 118.53 46.23) (end 117.14 47.62) (width 0.2) (layer "F.Cu") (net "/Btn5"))
 (segment (start 121.07 48.77) (end 118.58 51.26) (width 0.2) (layer "F.Cu") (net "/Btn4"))
 (segment (start 118.58 51.26) (end 118.58 65.5) (width 0.2) (layer "F.Cu") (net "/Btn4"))
 (segment (start 121.12 51.88) (end 122.22 50.78) (width 0.2) (layer "F.Cu") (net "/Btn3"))
 (segment (start 122.22 47.38) (end 121.07 46.23) (width 0.2) (layer "F.Cu") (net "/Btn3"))
 (segment (start 122.22 50.78) (end 122.22 47.38) (width 0.2) (layer "F.Cu") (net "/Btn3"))
 (segment (start 121.12 65.5) (end 121.12 51.88) (width 0.2) (layer "F.Cu") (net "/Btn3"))
 (segment (start 123.61 48.77) (end 123.61 65.45) (width 0.2) (layer "F.Cu") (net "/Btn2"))
 (segment (start 123.61 65.45) (end 123.66 65.5) (width 0.2) (layer "F.Cu") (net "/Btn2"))
 (segment (start 125 50) (end 125 47.38) (width 0.2) (layer "F.Cu") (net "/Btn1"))
 (segment (start 126.2 51.2) (end 125 50) (width 0.2) (layer "F.Cu") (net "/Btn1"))
 (segment (start 125 47.38) (end 126.15 46.23) (width 0.2) (layer "F.Cu") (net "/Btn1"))
 (segment (start 126.2 65.5) (end 126.2 51.2) (width 0.2) (layer "F.Cu") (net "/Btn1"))
 (segment (start 130.08 51.58) (end 130.08 48.293654) (width 0.2) (layer "F.Cu") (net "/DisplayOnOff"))
 (segment (start 130.5 52) (end 130.08 51.58) (width 0.2) (layer "F.Cu") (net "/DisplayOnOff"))
 (segment (start 130.08 48.293654) (end 130.993654 47.38) (width 0.2) (layer "F.Cu") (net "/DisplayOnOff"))
 (segment (start 132.62 47.38) (end 133.77 46.23) (width 0.2) (layer "F.Cu") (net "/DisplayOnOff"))
 (segment (start 130.993654 47.38) (end 132.62 47.38) (width 0.2) (layer "F.Cu") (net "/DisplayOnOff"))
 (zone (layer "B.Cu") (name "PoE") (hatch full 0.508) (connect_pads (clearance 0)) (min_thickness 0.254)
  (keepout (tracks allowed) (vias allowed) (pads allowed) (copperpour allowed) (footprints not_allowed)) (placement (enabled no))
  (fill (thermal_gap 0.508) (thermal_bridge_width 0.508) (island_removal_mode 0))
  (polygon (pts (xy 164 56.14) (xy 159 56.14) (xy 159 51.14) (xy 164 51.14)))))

